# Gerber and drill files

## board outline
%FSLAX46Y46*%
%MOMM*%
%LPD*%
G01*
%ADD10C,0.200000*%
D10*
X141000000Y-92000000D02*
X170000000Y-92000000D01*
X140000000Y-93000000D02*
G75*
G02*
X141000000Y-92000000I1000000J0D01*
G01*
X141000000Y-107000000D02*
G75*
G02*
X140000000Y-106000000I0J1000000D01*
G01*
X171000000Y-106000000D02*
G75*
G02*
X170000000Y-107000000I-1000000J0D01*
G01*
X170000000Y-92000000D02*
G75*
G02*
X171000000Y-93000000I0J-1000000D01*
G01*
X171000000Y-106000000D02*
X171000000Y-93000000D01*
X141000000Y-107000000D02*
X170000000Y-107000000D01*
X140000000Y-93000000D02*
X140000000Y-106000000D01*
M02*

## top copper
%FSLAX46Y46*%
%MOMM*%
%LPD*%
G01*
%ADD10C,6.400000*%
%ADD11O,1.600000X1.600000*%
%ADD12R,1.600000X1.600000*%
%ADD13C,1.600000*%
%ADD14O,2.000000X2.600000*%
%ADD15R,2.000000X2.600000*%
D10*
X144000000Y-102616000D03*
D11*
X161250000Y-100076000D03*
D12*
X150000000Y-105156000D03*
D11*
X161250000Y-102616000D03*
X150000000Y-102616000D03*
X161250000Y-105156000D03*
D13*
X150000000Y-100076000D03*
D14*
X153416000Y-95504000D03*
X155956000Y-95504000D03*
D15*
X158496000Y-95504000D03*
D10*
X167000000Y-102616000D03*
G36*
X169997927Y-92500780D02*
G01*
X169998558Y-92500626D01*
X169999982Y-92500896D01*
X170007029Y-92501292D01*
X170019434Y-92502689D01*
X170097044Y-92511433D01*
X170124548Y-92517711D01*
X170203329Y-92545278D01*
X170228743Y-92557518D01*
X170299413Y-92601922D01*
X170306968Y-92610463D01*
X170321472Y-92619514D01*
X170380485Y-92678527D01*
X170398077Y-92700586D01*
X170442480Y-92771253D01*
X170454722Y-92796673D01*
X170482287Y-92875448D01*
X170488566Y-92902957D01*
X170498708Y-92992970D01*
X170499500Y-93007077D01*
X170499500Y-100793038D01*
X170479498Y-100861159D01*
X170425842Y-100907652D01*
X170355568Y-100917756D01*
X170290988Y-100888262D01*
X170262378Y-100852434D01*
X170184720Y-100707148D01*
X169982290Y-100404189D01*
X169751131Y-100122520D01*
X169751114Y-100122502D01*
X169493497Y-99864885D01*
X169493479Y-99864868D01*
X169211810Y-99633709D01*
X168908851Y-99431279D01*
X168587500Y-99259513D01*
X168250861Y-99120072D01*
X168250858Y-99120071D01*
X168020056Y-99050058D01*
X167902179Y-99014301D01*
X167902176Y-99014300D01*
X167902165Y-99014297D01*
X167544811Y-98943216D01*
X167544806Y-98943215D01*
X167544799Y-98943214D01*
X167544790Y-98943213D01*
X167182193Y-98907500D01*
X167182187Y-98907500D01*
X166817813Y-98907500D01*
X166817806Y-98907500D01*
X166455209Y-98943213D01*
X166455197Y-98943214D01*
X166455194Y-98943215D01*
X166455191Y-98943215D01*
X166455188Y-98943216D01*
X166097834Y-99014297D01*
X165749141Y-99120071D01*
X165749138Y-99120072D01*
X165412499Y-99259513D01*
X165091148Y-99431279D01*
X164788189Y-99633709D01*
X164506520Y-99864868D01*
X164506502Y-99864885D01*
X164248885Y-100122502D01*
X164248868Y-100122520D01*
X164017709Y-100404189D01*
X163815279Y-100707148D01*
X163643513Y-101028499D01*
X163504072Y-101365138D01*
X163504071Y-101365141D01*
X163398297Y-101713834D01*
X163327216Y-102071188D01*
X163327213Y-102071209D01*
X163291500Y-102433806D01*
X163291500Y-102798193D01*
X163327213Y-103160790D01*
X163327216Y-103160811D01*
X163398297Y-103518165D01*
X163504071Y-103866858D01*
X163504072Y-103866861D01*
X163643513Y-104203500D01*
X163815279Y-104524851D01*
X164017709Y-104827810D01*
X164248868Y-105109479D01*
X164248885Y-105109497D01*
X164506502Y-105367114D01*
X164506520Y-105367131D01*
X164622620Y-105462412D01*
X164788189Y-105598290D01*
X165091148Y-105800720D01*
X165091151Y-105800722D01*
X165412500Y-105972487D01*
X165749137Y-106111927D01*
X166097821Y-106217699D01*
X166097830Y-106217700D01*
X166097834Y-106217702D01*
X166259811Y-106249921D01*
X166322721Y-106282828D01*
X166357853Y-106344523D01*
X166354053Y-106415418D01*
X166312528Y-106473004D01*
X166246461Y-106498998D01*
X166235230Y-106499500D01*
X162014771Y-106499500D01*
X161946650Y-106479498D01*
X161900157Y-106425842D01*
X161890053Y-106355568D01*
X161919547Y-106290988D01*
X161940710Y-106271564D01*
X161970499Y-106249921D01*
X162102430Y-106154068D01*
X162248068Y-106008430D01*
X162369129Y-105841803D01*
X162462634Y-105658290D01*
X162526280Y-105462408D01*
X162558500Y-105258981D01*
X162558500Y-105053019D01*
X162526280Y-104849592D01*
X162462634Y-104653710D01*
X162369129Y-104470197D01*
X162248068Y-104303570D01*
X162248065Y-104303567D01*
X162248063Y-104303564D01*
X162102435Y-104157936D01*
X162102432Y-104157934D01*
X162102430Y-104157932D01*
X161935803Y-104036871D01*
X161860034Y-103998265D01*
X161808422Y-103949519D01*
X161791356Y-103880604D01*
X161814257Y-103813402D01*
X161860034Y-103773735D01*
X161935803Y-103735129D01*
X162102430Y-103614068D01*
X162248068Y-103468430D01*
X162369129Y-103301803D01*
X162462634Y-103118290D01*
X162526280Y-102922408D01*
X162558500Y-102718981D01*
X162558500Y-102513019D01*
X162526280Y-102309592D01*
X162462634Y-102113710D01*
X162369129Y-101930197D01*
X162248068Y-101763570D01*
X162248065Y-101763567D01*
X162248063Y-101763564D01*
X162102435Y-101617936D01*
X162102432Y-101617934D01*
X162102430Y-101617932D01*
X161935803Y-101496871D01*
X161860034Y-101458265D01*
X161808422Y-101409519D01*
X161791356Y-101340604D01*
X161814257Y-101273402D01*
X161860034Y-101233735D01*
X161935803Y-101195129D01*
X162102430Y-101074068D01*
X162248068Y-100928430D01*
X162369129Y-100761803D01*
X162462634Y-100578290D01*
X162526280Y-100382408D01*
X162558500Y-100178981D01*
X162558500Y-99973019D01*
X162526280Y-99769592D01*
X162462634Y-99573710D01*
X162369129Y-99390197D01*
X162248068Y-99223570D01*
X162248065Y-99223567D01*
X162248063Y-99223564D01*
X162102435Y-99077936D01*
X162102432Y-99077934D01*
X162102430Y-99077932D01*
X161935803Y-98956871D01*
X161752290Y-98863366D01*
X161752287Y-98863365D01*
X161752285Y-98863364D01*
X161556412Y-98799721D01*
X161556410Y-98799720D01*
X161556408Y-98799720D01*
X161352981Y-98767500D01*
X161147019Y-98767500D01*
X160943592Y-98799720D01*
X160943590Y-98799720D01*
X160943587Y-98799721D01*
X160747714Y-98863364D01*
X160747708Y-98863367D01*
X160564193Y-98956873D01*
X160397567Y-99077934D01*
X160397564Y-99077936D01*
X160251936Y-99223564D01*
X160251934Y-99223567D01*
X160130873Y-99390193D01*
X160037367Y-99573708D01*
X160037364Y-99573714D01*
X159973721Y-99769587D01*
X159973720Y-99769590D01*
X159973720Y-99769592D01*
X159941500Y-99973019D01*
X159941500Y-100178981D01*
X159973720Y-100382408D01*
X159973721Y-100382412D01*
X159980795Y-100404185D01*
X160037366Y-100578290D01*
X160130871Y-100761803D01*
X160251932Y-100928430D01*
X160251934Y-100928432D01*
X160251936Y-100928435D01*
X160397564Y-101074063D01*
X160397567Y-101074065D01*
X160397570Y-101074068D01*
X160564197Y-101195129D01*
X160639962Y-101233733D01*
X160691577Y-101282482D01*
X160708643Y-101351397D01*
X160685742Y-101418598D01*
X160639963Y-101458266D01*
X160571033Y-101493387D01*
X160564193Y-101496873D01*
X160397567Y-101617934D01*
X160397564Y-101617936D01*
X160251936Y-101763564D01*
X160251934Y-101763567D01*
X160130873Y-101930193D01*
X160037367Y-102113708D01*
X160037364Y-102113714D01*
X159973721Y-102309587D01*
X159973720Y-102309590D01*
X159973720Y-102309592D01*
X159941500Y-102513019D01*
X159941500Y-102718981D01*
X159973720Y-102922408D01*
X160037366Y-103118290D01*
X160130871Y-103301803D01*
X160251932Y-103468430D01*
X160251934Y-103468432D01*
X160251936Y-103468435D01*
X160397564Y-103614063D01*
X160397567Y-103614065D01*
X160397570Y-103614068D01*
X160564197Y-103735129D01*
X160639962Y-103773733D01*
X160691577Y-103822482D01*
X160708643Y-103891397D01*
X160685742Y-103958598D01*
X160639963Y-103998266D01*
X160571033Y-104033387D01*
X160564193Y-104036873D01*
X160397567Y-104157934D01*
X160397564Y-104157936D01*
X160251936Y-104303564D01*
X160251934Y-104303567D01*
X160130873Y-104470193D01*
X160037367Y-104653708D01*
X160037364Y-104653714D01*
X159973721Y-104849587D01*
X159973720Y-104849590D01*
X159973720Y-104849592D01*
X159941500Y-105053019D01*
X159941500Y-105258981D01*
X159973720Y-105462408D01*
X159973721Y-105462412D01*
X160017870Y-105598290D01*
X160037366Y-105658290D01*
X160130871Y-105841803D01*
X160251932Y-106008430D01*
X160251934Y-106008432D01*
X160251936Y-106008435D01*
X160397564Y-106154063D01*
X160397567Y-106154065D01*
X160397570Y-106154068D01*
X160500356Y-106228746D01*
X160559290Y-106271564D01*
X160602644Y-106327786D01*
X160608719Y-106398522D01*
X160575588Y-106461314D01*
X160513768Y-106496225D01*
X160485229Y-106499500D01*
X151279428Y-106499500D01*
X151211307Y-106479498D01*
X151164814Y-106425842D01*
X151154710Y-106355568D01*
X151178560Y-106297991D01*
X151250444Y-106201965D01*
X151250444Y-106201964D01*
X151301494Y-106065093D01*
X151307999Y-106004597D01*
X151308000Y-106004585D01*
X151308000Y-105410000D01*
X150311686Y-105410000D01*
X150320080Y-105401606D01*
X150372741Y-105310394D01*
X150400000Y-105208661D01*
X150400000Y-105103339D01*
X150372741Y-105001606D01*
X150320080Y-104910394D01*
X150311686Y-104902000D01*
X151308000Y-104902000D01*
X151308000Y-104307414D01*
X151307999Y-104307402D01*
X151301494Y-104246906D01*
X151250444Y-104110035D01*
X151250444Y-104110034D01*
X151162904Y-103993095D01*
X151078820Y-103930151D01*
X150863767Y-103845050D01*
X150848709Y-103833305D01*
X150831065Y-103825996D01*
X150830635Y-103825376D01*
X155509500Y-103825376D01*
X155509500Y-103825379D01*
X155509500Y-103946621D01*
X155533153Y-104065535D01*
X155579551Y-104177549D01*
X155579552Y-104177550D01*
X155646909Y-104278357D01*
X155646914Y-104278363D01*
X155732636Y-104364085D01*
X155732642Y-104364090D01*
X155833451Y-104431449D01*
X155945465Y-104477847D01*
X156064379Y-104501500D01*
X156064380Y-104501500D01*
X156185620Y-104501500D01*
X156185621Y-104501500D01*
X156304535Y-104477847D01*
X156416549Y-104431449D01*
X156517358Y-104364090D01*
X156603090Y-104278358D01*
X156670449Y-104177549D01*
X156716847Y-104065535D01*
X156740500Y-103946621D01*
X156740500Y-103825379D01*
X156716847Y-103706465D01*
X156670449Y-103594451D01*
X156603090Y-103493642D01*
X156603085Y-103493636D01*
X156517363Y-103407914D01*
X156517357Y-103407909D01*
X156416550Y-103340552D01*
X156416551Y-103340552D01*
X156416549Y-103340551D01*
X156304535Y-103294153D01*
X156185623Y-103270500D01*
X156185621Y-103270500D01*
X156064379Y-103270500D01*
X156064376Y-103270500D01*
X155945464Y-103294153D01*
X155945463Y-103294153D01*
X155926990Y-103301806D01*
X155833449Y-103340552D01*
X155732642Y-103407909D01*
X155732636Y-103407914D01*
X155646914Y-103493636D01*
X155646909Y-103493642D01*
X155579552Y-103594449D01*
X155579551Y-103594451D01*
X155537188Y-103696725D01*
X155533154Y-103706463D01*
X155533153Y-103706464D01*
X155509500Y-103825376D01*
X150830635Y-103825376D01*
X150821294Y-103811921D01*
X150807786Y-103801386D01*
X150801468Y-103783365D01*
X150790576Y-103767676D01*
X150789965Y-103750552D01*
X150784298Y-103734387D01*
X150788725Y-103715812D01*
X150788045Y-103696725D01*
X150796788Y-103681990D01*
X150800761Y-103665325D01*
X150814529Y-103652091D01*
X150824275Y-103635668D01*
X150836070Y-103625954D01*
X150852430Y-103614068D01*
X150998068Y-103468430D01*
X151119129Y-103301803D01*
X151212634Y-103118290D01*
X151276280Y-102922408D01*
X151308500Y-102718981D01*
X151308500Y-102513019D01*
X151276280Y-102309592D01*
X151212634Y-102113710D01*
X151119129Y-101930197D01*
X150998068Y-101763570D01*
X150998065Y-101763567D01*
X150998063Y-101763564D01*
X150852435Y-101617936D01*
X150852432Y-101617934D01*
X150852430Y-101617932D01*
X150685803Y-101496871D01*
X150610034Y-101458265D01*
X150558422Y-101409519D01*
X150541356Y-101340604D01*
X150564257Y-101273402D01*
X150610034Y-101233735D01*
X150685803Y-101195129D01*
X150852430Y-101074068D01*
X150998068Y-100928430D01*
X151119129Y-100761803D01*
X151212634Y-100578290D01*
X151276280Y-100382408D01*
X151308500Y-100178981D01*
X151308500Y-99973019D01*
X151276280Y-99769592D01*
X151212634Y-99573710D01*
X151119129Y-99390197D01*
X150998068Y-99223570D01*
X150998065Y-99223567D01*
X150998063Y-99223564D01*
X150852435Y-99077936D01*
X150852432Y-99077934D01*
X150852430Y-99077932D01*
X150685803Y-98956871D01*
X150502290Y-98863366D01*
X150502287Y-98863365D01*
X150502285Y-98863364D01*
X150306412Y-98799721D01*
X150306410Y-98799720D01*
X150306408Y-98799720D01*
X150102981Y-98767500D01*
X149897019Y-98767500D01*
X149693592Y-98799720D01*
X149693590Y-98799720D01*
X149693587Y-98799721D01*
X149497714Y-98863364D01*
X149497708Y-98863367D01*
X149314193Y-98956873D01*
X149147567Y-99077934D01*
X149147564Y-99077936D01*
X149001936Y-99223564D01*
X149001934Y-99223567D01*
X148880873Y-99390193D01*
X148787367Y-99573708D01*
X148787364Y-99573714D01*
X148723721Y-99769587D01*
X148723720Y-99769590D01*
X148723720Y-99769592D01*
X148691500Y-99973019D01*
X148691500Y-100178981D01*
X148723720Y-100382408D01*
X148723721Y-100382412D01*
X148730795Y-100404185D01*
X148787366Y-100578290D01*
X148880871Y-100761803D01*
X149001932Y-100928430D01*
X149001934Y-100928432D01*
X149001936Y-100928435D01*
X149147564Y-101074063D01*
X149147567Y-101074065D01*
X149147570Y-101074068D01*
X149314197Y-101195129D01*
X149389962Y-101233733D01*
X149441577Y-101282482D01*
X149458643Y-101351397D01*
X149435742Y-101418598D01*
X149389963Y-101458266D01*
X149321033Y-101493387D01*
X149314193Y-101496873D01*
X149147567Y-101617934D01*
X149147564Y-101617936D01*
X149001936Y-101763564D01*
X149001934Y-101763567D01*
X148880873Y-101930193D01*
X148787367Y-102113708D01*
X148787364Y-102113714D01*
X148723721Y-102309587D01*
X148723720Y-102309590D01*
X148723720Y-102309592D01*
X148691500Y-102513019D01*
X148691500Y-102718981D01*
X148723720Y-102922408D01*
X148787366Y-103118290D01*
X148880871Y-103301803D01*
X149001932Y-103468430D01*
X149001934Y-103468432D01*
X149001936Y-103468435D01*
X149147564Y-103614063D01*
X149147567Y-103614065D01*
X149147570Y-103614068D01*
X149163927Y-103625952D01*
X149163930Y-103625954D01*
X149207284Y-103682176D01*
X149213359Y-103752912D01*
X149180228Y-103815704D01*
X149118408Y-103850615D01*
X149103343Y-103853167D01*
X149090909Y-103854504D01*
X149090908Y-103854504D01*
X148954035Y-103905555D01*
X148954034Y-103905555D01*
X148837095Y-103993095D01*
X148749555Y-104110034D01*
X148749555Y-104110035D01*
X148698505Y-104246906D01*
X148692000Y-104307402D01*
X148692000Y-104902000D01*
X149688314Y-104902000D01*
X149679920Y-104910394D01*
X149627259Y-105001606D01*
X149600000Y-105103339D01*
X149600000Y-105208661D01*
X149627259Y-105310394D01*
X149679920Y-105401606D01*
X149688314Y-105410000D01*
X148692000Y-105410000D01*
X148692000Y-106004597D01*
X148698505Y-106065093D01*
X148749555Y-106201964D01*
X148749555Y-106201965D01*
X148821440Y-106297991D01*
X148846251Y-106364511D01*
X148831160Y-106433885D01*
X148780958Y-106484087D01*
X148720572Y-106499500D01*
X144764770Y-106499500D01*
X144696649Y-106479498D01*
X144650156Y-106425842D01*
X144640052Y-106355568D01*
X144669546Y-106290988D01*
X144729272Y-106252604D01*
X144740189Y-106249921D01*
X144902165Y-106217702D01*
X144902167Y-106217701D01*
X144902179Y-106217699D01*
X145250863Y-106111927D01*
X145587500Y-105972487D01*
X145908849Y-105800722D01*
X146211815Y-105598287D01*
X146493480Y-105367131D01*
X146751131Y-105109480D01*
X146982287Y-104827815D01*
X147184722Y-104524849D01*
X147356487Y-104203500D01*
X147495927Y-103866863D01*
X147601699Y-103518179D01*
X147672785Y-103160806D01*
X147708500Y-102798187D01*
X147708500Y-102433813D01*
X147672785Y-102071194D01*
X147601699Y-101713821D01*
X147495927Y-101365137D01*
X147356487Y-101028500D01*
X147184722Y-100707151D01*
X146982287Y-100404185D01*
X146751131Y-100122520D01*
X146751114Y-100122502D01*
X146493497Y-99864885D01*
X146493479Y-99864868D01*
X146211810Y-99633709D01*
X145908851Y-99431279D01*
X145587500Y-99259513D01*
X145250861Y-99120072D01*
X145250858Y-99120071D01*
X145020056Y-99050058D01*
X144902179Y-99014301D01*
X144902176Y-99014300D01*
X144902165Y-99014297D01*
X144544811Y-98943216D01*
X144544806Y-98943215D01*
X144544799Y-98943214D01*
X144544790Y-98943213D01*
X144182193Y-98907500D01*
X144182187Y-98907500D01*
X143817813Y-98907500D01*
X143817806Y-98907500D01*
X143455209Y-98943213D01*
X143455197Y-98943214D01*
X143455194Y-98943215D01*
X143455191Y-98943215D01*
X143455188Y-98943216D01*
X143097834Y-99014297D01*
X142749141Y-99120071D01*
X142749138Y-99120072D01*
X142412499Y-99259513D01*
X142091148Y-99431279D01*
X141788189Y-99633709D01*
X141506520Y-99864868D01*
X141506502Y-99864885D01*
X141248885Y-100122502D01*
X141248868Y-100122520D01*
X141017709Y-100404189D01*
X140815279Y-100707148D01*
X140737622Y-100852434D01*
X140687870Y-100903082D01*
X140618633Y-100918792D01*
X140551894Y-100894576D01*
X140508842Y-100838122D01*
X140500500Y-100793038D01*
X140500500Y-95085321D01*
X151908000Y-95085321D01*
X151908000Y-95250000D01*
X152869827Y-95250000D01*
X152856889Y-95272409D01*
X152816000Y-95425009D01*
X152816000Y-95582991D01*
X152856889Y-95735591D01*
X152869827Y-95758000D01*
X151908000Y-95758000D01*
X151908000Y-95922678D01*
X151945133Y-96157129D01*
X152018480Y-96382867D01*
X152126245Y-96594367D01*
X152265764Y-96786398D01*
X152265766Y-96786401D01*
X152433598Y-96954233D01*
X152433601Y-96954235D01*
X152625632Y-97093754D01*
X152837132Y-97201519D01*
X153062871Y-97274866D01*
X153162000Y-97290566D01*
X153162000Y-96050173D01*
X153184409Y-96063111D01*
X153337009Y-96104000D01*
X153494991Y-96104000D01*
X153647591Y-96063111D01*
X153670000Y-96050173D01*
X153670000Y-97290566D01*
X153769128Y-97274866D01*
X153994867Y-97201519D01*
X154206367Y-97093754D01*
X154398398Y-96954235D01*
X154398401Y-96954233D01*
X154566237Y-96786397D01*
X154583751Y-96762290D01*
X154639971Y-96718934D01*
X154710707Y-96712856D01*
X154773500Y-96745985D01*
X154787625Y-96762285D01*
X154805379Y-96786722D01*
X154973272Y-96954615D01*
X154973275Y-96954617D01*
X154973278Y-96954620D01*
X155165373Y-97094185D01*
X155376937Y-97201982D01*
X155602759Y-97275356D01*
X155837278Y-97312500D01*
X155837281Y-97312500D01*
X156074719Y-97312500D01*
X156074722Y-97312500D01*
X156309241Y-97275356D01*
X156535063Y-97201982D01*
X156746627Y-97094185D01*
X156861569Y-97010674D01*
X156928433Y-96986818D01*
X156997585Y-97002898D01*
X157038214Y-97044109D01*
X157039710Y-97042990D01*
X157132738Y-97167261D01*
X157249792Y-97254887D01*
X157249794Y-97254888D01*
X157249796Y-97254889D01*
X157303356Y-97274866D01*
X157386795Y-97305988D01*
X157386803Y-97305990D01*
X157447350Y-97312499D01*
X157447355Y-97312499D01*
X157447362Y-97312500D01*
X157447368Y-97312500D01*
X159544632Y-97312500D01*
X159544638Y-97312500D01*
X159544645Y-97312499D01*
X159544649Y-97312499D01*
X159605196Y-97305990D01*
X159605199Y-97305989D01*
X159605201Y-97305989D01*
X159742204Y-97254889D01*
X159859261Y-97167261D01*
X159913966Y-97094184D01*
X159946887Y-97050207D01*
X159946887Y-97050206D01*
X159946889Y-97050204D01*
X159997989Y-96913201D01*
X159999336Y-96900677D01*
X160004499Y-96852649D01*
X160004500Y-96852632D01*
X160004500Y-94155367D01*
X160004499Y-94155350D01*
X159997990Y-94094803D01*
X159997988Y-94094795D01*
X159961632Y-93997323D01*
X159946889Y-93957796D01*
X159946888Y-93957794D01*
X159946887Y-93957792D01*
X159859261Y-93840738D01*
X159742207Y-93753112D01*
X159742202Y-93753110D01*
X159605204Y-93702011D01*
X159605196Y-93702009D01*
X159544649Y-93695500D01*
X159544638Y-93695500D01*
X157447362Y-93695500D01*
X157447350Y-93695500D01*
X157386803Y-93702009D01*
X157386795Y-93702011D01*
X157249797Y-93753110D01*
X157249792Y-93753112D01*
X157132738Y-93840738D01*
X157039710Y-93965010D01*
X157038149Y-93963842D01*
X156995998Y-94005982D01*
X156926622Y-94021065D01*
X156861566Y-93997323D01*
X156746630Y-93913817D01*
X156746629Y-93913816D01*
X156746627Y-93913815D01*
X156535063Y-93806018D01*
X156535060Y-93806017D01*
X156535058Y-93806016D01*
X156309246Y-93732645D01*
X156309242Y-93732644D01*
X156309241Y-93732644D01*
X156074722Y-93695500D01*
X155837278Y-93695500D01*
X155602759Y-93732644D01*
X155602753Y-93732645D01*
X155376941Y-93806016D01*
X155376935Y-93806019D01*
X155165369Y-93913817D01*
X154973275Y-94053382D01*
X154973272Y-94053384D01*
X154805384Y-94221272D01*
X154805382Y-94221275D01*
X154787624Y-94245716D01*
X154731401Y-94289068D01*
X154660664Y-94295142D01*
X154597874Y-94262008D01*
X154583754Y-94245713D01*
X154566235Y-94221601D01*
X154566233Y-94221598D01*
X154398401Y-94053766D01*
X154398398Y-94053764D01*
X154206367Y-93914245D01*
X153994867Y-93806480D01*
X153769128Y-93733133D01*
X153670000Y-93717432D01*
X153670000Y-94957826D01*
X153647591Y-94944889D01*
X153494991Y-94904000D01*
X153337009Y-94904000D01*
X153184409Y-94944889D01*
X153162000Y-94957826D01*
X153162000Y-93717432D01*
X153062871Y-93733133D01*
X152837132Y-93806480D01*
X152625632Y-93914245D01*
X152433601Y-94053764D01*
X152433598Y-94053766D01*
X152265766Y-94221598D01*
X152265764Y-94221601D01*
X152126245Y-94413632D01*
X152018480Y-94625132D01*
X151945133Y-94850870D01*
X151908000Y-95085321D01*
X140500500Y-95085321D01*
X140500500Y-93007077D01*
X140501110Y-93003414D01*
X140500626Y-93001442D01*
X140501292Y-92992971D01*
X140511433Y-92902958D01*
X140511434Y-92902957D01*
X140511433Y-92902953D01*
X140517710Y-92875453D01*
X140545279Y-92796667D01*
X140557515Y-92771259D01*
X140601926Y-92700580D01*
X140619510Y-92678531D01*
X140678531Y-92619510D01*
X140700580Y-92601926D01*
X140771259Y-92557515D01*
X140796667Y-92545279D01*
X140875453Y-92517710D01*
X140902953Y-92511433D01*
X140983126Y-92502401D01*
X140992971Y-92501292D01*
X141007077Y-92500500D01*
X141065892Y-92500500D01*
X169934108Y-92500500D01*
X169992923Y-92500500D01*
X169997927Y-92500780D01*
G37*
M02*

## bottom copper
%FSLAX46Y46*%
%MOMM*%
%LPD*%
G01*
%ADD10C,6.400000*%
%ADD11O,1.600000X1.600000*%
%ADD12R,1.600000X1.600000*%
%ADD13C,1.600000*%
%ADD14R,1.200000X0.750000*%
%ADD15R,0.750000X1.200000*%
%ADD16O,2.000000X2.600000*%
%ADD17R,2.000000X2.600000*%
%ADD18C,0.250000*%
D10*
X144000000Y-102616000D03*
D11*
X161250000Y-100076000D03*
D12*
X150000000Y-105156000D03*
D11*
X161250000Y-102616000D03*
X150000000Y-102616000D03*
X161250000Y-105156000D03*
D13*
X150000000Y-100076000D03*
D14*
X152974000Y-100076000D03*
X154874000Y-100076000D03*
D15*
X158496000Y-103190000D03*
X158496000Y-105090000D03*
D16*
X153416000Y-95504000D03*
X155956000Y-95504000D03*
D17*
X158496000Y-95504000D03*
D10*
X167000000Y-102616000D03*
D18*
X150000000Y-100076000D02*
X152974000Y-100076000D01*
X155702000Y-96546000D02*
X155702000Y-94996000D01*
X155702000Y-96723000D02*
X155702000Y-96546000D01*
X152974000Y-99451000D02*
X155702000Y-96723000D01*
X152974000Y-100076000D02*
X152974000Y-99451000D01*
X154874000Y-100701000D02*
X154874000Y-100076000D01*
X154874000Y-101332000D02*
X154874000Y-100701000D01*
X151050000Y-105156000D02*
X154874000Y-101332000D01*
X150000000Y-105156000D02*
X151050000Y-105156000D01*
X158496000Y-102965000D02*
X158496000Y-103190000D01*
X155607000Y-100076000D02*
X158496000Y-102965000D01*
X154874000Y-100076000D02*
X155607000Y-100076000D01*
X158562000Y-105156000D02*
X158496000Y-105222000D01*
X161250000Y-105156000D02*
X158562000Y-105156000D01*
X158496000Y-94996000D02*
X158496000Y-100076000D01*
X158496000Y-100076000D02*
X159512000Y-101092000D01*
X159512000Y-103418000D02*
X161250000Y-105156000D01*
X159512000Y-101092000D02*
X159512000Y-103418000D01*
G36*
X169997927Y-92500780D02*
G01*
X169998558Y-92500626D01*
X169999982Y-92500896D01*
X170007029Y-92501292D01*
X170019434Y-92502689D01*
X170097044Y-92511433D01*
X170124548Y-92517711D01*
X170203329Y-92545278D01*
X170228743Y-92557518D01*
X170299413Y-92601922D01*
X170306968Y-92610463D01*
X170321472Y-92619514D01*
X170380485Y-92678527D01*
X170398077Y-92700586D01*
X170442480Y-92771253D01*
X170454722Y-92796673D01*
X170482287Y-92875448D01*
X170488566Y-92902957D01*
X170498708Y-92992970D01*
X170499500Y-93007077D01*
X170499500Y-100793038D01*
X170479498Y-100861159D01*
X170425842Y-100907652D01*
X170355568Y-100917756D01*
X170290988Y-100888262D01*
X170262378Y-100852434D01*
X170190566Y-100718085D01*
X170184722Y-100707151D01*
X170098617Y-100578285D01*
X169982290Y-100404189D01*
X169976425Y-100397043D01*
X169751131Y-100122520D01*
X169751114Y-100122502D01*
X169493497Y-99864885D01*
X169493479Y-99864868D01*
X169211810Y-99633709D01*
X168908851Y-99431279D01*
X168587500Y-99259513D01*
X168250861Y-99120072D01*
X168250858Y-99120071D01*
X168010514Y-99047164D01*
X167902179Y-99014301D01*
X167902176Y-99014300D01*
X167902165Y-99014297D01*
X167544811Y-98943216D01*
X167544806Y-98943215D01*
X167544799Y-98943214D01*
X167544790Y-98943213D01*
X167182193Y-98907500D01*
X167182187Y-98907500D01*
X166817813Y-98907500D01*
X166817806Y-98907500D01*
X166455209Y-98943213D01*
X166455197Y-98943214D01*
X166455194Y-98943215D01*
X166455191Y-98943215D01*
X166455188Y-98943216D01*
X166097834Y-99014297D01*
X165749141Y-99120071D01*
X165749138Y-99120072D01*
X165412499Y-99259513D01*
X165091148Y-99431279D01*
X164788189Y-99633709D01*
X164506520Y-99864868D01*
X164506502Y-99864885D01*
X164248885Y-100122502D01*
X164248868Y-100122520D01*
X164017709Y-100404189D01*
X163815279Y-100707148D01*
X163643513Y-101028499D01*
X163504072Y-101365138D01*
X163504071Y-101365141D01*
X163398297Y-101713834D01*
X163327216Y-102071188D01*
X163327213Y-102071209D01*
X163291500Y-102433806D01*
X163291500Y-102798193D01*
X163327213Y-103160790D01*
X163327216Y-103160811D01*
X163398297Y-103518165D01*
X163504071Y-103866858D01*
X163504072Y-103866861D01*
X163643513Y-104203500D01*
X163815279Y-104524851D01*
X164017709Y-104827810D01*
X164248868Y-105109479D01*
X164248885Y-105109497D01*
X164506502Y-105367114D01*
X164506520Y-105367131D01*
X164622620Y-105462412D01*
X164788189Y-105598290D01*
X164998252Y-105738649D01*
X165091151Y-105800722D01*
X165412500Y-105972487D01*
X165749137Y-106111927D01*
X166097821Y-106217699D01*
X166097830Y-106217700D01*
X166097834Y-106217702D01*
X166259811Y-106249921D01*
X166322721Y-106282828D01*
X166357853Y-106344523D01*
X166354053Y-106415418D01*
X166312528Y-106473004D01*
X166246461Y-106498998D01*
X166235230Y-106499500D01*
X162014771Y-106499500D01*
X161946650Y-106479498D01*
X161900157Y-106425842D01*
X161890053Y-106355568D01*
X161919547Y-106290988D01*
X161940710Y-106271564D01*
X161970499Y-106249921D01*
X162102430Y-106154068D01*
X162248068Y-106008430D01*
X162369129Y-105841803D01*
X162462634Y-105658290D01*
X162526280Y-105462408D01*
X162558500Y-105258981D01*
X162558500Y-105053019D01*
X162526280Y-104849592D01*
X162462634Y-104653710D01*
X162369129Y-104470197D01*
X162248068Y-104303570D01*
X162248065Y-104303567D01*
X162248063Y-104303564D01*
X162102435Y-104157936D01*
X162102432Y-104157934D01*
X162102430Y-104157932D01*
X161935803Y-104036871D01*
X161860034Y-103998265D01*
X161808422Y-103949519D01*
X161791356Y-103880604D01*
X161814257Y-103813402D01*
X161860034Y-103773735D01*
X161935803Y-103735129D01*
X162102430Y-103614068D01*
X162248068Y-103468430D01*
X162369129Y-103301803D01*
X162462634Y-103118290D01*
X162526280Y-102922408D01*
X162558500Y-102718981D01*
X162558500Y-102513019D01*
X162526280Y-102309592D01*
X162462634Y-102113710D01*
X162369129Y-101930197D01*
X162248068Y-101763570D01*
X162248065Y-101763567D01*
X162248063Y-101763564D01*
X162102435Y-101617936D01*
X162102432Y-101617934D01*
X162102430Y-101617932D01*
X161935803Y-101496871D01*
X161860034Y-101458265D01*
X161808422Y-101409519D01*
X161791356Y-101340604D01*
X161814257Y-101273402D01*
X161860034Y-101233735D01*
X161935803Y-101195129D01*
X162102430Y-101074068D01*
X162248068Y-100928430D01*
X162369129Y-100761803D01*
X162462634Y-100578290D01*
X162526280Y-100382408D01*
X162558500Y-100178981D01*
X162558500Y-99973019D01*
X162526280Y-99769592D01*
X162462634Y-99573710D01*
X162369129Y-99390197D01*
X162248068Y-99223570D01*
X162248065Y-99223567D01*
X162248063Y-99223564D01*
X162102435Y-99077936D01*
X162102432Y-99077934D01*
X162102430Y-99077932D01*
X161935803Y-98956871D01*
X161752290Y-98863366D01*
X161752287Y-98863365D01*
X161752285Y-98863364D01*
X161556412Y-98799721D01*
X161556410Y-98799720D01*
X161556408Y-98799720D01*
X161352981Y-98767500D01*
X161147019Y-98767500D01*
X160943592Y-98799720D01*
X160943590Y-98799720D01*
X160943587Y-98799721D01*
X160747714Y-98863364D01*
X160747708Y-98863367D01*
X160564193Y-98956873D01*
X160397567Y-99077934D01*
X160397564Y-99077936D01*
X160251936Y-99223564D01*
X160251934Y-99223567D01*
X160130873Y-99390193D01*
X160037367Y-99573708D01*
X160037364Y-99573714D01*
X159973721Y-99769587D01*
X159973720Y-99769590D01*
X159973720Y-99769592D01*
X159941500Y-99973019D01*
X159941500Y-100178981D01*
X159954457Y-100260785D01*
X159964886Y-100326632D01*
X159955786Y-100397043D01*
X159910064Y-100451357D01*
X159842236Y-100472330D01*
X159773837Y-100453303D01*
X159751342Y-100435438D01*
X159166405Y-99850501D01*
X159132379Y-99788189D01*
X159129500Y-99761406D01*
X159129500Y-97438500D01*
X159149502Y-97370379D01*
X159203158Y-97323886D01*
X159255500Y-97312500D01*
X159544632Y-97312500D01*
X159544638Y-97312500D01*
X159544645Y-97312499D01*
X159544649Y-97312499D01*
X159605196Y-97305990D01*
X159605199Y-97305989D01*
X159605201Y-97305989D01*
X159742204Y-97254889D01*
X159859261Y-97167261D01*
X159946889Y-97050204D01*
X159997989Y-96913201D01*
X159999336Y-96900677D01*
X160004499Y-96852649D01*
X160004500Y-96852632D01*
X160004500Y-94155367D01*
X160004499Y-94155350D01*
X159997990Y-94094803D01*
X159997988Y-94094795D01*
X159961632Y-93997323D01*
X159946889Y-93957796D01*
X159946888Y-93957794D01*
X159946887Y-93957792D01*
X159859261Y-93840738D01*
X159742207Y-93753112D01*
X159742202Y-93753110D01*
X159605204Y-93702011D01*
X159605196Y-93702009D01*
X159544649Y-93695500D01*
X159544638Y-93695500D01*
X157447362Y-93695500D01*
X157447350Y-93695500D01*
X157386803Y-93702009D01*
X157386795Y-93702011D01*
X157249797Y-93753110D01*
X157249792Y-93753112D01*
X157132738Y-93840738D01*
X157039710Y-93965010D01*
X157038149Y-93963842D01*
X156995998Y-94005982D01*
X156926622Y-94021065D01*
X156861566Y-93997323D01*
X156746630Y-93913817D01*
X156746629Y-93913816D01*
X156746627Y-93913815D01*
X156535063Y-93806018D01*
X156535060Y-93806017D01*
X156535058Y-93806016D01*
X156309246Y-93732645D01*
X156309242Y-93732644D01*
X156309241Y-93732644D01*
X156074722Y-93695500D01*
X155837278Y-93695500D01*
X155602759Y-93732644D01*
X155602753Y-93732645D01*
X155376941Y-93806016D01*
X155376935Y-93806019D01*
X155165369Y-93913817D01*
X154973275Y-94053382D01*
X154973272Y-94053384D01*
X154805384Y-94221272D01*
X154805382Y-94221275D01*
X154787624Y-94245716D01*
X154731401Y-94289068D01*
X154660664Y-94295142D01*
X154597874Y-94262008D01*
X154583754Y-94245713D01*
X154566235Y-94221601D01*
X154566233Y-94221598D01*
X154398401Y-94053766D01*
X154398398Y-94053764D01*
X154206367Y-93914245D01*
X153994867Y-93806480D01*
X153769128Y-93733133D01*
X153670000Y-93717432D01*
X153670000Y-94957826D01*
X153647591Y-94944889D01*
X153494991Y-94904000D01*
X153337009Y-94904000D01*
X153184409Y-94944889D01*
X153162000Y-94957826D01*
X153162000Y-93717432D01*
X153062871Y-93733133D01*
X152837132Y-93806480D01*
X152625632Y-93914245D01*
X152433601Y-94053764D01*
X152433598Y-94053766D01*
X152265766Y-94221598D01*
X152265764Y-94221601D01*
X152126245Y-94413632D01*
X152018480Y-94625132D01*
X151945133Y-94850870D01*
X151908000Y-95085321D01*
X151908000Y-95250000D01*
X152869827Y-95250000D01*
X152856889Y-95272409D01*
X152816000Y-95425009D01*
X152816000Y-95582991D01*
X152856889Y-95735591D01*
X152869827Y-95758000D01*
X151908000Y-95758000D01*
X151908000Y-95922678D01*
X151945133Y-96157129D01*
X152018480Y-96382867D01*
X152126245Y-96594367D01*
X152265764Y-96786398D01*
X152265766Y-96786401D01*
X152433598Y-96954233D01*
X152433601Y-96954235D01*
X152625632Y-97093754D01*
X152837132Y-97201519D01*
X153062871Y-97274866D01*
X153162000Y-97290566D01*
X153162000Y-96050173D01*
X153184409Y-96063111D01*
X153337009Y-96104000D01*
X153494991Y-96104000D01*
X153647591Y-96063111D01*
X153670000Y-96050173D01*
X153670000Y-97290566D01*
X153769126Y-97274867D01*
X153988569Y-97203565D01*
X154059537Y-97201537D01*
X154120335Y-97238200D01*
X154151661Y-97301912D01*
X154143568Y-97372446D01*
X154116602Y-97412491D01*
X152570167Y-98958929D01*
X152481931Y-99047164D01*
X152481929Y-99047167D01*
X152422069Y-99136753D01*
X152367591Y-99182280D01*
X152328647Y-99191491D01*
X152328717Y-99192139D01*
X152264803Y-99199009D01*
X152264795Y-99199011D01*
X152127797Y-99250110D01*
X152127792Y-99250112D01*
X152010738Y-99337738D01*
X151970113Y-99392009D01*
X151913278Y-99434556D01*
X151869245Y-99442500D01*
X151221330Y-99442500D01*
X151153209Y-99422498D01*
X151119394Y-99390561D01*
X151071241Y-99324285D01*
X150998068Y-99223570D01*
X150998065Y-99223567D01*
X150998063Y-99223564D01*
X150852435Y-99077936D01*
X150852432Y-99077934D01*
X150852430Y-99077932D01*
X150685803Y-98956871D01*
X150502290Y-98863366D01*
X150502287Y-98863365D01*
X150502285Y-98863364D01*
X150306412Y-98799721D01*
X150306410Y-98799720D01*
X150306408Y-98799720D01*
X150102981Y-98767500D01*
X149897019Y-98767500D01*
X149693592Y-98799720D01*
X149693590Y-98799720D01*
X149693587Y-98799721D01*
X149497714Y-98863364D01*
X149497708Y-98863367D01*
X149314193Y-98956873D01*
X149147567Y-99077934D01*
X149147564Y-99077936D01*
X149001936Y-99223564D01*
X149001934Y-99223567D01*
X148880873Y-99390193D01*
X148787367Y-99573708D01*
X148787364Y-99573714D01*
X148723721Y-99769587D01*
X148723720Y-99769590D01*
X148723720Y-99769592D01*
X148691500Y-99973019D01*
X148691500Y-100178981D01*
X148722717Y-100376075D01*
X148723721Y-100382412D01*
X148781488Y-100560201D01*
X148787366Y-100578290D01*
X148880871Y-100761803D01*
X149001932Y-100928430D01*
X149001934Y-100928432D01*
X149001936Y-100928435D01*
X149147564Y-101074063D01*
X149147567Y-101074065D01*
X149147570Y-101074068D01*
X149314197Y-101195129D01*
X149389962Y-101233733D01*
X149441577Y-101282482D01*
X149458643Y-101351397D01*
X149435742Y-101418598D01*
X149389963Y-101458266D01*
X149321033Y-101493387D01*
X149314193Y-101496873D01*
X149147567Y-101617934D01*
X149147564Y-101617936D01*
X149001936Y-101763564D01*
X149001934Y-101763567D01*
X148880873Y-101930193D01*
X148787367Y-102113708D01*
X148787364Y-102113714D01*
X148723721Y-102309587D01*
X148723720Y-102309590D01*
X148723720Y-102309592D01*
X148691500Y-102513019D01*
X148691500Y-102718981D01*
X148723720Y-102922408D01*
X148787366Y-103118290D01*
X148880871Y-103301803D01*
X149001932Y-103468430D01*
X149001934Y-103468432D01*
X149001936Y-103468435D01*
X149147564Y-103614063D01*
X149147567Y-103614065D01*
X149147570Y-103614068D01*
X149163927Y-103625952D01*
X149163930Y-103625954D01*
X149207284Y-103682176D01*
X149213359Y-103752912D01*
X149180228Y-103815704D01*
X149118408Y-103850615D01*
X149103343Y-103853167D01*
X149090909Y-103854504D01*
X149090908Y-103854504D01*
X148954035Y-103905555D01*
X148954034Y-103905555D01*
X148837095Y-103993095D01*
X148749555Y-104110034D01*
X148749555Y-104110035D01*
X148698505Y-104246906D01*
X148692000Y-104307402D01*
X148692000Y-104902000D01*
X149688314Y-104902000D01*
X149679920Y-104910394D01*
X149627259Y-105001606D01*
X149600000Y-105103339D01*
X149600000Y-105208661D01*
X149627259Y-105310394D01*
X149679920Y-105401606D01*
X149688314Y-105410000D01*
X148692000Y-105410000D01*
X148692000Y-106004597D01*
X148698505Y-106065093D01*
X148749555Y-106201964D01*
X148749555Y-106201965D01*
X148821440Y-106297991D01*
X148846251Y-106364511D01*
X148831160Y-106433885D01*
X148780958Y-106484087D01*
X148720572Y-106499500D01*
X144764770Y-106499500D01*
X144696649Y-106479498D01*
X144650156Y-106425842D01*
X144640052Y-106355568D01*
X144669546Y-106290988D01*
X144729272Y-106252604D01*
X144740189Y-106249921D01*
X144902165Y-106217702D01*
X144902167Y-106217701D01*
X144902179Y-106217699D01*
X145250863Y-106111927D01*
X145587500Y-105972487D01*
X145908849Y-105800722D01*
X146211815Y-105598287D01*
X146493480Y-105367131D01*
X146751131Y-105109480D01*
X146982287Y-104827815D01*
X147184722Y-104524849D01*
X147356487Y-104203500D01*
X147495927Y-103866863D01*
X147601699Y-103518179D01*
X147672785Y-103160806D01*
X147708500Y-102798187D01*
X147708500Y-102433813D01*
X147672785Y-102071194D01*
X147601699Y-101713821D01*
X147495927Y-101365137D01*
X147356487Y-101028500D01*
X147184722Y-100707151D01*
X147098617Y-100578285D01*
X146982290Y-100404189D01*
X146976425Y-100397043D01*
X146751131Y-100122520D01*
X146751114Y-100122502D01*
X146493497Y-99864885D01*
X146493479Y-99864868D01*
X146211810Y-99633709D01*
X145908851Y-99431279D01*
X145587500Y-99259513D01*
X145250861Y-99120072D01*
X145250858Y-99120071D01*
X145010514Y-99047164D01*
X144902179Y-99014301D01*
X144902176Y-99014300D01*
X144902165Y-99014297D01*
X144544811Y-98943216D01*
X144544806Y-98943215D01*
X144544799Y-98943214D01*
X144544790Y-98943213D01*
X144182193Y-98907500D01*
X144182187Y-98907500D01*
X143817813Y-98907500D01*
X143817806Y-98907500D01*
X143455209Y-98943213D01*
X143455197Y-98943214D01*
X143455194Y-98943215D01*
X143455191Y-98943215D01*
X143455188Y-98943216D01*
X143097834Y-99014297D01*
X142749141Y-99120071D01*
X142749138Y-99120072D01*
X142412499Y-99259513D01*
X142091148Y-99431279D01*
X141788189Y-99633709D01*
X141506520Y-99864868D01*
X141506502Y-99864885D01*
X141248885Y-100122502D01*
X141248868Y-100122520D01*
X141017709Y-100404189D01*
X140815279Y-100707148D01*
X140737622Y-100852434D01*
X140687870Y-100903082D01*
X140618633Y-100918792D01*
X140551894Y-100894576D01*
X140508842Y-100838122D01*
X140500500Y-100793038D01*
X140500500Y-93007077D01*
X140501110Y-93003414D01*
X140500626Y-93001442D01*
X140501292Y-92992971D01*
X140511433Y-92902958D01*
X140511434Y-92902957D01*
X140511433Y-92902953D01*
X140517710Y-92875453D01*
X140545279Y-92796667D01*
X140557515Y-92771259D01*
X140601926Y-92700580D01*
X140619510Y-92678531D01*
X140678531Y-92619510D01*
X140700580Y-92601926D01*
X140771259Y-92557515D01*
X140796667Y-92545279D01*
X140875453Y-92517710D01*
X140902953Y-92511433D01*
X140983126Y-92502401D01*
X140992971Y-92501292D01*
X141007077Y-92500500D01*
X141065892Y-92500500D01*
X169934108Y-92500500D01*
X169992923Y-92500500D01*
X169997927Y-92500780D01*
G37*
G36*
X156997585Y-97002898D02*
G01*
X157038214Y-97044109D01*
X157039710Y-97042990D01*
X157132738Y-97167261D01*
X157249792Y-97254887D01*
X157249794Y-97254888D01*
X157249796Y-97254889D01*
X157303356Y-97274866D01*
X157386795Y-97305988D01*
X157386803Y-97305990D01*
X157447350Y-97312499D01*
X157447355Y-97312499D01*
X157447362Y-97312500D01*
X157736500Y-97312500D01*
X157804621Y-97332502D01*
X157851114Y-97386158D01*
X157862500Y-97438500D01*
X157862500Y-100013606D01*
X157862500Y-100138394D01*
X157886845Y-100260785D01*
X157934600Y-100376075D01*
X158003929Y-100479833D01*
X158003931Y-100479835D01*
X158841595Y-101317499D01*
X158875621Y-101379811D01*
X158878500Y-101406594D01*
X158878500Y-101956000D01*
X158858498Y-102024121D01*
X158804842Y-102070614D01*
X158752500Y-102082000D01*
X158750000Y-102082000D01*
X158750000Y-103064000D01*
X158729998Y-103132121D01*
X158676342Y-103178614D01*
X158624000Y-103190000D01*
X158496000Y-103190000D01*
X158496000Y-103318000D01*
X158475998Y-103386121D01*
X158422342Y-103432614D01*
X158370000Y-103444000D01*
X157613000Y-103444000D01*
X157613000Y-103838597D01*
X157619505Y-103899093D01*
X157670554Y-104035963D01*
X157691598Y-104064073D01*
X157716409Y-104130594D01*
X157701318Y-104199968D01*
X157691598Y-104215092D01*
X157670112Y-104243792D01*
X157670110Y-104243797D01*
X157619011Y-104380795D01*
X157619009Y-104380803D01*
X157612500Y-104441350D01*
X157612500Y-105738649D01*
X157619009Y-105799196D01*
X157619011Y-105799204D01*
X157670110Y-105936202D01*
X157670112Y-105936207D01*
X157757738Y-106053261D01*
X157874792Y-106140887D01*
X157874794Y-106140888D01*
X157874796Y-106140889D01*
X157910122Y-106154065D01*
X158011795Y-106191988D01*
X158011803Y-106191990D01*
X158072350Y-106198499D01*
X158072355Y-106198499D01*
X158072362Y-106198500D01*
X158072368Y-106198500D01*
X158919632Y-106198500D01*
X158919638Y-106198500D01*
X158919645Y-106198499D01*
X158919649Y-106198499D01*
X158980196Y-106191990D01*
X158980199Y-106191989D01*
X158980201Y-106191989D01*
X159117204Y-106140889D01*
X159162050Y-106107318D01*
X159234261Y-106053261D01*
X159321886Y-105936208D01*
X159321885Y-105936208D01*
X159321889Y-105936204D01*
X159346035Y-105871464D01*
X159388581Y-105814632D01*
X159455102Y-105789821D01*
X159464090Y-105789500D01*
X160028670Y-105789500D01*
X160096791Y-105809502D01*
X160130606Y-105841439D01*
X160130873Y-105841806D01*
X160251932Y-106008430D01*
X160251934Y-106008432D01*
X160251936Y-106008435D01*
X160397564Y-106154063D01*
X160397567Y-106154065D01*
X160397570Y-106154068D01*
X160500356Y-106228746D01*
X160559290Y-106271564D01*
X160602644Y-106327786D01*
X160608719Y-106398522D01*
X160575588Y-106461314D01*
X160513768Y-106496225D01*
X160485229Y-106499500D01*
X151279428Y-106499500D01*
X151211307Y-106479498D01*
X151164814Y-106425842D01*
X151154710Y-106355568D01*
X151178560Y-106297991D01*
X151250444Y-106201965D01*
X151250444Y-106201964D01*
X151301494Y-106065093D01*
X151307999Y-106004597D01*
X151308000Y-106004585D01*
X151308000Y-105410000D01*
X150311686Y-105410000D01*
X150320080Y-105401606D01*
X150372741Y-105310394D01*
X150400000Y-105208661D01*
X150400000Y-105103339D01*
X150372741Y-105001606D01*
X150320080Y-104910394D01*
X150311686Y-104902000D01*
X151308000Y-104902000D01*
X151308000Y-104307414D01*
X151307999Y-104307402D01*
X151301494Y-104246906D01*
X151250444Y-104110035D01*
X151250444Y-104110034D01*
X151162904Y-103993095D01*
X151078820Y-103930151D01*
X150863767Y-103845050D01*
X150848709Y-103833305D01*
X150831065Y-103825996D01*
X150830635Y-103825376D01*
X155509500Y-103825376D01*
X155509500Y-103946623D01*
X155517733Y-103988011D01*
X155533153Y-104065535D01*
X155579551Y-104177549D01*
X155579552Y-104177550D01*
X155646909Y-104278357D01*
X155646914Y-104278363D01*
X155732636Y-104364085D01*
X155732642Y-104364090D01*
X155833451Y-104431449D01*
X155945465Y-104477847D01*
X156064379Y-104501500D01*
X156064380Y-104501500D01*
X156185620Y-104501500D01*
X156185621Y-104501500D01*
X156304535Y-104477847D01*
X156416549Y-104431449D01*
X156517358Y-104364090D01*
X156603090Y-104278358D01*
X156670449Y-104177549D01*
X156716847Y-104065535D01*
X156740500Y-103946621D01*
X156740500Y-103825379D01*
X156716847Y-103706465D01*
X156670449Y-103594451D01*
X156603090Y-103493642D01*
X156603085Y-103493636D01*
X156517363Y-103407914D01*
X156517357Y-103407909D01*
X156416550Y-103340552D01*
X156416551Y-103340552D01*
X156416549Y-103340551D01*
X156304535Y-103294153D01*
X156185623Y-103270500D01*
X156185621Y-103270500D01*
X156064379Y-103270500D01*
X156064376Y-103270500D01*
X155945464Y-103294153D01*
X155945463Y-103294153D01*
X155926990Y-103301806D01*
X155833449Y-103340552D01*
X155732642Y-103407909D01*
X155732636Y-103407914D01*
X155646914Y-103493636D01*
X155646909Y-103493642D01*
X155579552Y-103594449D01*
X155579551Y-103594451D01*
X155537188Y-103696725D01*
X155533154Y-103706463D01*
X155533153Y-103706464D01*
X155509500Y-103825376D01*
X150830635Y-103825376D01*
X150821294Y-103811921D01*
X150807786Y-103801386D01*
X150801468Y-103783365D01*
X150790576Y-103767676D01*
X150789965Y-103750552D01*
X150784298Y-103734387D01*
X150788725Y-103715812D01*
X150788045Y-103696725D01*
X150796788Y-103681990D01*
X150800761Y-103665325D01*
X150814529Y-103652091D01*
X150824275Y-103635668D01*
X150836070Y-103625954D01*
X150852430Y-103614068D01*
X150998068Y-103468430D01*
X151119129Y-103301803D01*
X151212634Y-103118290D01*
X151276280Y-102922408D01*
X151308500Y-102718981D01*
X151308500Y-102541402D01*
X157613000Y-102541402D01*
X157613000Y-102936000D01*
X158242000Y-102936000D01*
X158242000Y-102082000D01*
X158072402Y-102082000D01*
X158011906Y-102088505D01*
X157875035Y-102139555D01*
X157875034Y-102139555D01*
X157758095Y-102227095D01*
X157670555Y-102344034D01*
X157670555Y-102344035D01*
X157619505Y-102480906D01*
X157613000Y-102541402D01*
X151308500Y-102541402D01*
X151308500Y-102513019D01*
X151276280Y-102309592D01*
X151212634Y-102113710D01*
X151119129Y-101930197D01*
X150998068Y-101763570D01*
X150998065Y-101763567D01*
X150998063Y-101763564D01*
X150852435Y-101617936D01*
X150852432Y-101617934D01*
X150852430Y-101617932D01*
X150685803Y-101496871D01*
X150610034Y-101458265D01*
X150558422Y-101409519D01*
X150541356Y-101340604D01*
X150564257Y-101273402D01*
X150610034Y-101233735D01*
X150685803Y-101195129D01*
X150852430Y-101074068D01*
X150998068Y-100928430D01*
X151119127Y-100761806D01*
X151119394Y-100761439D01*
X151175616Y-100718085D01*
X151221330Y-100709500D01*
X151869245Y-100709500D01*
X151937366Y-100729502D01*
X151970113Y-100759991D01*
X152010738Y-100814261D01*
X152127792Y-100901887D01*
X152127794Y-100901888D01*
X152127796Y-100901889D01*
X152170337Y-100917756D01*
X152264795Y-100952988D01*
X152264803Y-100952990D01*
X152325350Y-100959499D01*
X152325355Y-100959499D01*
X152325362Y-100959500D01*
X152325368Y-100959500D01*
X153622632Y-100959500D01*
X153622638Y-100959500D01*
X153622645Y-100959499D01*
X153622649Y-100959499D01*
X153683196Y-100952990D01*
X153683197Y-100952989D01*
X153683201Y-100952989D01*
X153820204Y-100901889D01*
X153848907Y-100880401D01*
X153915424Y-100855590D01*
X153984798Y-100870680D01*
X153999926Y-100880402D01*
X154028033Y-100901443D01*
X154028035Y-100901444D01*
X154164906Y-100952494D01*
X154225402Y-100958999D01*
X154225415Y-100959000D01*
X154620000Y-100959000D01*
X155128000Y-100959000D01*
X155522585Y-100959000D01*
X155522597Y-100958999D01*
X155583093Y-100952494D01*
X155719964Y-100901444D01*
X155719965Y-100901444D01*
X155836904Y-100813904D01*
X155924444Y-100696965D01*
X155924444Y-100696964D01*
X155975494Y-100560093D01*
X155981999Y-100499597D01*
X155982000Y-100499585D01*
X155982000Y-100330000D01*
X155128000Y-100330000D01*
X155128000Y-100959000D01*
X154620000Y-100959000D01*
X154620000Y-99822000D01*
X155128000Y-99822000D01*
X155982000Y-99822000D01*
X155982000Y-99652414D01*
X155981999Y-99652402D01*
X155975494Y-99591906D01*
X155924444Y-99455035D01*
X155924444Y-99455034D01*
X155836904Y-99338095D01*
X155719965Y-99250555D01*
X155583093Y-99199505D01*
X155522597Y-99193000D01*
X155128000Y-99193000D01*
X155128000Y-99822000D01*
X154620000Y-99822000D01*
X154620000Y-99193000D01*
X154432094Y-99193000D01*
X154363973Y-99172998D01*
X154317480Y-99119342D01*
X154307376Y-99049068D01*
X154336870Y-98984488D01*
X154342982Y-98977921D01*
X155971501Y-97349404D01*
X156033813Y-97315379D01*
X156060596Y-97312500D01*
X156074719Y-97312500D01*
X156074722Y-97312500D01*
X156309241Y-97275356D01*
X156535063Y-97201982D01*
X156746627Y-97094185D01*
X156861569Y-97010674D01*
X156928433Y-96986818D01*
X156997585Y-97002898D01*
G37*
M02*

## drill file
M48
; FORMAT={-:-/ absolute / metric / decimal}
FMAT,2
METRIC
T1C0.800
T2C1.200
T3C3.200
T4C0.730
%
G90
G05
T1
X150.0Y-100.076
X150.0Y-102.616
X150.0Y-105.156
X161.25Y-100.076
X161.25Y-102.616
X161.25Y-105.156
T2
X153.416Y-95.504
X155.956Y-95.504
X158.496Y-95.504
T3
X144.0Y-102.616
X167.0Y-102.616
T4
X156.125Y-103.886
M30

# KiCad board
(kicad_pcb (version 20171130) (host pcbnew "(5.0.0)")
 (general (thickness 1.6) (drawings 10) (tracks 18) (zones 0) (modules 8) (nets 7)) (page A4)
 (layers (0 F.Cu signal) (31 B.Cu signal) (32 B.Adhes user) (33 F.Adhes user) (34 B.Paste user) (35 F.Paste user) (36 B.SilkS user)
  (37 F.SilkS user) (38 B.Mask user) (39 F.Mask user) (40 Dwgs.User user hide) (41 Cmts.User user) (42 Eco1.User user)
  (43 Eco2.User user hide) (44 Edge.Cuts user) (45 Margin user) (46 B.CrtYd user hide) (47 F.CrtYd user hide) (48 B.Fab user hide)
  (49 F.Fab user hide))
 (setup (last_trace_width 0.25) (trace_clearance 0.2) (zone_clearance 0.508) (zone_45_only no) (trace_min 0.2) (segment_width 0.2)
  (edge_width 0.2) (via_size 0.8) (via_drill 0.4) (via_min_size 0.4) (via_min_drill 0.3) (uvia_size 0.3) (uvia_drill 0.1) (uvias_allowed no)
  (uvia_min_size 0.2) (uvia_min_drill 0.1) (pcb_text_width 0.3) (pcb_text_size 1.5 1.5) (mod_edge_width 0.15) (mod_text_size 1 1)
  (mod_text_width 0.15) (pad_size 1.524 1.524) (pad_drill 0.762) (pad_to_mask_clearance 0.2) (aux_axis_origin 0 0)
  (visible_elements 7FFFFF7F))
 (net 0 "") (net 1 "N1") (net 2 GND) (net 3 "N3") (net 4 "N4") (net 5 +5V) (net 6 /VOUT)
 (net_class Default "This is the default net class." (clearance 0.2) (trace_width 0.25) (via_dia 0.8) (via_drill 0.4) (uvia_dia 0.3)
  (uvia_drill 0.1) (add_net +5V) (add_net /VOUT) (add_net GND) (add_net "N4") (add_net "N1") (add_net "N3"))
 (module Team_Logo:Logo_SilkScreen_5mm (layer B.Cu) (at 144.272 95.504 180)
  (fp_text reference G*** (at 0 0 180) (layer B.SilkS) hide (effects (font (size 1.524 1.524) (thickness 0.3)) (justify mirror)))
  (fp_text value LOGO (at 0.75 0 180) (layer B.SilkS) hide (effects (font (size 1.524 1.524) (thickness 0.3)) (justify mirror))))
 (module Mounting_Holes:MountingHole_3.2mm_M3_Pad (layer F.Cu) (at 144 102.616)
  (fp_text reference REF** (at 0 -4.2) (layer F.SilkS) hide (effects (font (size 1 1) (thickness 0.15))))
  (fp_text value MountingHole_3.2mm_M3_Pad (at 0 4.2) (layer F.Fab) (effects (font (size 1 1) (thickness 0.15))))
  (pad 1 thru_hole circle (at 0 0) (size 6.4 6.4) (drill 3.2) (layers *.Cu *.Mask)))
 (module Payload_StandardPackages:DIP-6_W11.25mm (layer F.Cu) (at 150 100.076)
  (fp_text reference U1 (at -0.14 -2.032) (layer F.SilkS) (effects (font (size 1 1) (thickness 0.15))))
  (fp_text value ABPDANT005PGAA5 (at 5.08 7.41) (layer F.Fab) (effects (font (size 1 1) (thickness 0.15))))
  (pad "" np_thru_hole circle (at 6.125 3.81) (size 0.73 0.73) (drill 0.73) (layers *.Cu *.Mask))
  (pad 4 thru_hole oval (at 11.25 0) (size 1.6 1.6) (drill 0.8) (layers *.Cu *.Mask) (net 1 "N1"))
  (pad 1 thru_hole rect (at 0 5.08) (size 1.6 1.6) (drill 0.8) (layers *.Cu *.Mask) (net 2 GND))
  (pad 5 thru_hole oval (at 11.25 2.54) (size 1.6 1.6) (drill 0.8) (layers *.Cu *.Mask) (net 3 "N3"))
  (pad 2 thru_hole oval (at 0 2.54) (size 1.6 1.6) (drill 0.8) (layers *.Cu *.Mask) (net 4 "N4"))
  (pad 6 thru_hole oval (at 11.25 5.08) (size 1.6 1.6) (drill 0.8) (layers *.Cu *.Mask) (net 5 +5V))
  (pad 3 thru_hole circle (at 0 0) (size 1.6 1.6) (drill 0.8) (layers *.Cu *.Mask) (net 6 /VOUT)))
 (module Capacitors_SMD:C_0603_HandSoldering (layer B.Cu) (at 153.924 100.076)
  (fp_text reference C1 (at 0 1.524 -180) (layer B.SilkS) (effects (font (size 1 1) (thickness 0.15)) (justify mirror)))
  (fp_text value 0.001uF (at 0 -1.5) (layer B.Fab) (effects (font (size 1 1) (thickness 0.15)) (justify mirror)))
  (pad 1 smd rect (at -0.95 0) (size 1.2 0.75) (layers B.Cu B.Paste B.Mask) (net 6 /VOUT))
  (pad 2 smd rect (at 0.95 0) (size 1.2 0.75) (layers B.Cu B.Paste B.Mask) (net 2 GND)))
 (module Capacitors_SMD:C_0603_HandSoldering (layer B.Cu) (at 158.496 104.14 90)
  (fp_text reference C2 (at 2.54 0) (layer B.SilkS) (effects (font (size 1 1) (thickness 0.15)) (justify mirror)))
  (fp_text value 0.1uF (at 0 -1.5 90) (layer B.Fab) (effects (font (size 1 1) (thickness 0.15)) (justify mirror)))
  (pad 2 smd rect (at 0.95 0 90) (size 1.2 0.75) (layers B.Cu B.Paste B.Mask) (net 2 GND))
  (pad 1 smd rect (at -0.95 0 90) (size 1.2 0.75) (layers B.Cu B.Paste B.Mask) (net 5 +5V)))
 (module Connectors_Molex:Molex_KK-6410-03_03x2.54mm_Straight (layer B.Cu) (at 158.496 95.504 180)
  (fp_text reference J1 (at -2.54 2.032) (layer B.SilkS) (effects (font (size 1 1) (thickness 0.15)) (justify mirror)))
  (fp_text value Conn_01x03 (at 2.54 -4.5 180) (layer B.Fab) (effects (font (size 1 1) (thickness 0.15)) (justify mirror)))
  (pad 3 thru_hole oval (at 5.08 0 180) (size 2 2.6) (drill 1.2) (layers *.Cu *.Mask) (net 2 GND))
  (pad 2 thru_hole oval (at 2.54 0 180) (size 2 2.6) (drill 1.2) (layers *.Cu *.Mask) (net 6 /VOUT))
  (pad 1 thru_hole rect (at 0 0 180) (size 2 2.6) (drill 1.2) (layers *.Cu *.Mask) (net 5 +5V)))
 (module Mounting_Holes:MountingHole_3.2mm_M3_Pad (layer F.Cu) (at 167 102.616)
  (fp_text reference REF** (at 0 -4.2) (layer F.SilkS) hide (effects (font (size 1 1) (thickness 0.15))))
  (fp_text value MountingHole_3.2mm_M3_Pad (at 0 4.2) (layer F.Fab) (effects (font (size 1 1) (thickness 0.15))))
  (pad 1 thru_hole circle (at 0 0) (size 6.4 6.4) (drill 3.2) (layers *.Cu *.Mask)))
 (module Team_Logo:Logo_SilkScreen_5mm (layer F.Cu) (at 167.132 95.504)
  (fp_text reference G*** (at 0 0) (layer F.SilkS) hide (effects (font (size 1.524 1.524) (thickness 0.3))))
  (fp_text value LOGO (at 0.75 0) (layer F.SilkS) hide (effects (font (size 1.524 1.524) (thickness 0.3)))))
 (gr_line (start 141 92) (end 170 92) (layer Edge.Cuts) (width 0.2))
 (gr_arc (start 141 93) (end 140 93) (angle 90) (layer Edge.Cuts) (width 0.2))
 (gr_arc (start 141 106) (end 140 106) (angle -90) (layer Edge.Cuts) (width 0.2))
 (gr_arc (start 170 106) (end 170 107) (angle -90) (layer Edge.Cuts) (width 0.2))
 (gr_arc (start 170 93) (end 171 93) (angle -90) (layer Edge.Cuts) (width 0.2))
 (gr_line (start 171 106) (end 171 93) (layer Edge.Cuts) (width 0.2))
 (gr_line (start 141 107) (end 170 107) (layer Edge.Cuts) (width 0.2))
 (gr_line (start 140 93) (end 140 106) (layer Edge.Cuts) (width 0.2))
 (segment (start 150 100.076) (end 152.974 100.076) (width 0.25) (layer B.Cu) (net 6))
 (segment (start 155.702 96.546) (end 155.702 94.996) (width 0.25) (layer B.Cu) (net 6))
 (segment (start 155.702 96.723) (end 155.702 96.546) (width 0.25) (layer B.Cu) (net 6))
 (segment (start 152.974 99.451) (end 155.702 96.723) (width 0.25) (layer B.Cu) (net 6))
 (segment (start 152.974 100.076) (end 152.974 99.451) (width 0.25) (layer B.Cu) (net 6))
 (segment (start 154.874 100.701) (end 154.874 100.076) (width 0.25) (layer B.Cu) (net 2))
 (segment (start 154.874 101.332) (end 154.874 100.701) (width 0.25) (layer B.Cu) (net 2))
 (segment (start 151.05 105.156) (end 154.874 101.332) (width 0.25) (layer B.Cu) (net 2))
 (segment (start 150 105.156) (end 151.05 105.156) (width 0.25) (layer B.Cu) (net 2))
 (segment (start 158.496 102.965) (end 158.496 103.19) (width 0.25) (layer B.Cu) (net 2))
 (segment (start 155.607 100.076) (end 158.496 102.965) (width 0.25) (layer B.Cu) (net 2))
 (segment (start 154.874 100.076) (end 155.607 100.076) (width 0.25) (layer B.Cu) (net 2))
 (segment (start 158.562 105.156) (end 158.496 105.222) (width 0.25) (layer B.Cu) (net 5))
 (segment (start 161.25 105.156) (end 158.562 105.156) (width 0.25) (layer B.Cu) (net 5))
 (segment (start 158.496 94.996) (end 158.496 100.076) (width 0.25) (layer B.Cu) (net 5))
 (segment (start 158.496 100.076) (end 159.512 101.092) (width 0.25) (layer B.Cu) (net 5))
 (segment (start 159.512 103.418) (end 161.25 105.156) (width 0.25) (layer B.Cu) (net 5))
 (segment (start 159.512 101.092) (end 159.512 103.418) (width 0.25) (layer B.Cu) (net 5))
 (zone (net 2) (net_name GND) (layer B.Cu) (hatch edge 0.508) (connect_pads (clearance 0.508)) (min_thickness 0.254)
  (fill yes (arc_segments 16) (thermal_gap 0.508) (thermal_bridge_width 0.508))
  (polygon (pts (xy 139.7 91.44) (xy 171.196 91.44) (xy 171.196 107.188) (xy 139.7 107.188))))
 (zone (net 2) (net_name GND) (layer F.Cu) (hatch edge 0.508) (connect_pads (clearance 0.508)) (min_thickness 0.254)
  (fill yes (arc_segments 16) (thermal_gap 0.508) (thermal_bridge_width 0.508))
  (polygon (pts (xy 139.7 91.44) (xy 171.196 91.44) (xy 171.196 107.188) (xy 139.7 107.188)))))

